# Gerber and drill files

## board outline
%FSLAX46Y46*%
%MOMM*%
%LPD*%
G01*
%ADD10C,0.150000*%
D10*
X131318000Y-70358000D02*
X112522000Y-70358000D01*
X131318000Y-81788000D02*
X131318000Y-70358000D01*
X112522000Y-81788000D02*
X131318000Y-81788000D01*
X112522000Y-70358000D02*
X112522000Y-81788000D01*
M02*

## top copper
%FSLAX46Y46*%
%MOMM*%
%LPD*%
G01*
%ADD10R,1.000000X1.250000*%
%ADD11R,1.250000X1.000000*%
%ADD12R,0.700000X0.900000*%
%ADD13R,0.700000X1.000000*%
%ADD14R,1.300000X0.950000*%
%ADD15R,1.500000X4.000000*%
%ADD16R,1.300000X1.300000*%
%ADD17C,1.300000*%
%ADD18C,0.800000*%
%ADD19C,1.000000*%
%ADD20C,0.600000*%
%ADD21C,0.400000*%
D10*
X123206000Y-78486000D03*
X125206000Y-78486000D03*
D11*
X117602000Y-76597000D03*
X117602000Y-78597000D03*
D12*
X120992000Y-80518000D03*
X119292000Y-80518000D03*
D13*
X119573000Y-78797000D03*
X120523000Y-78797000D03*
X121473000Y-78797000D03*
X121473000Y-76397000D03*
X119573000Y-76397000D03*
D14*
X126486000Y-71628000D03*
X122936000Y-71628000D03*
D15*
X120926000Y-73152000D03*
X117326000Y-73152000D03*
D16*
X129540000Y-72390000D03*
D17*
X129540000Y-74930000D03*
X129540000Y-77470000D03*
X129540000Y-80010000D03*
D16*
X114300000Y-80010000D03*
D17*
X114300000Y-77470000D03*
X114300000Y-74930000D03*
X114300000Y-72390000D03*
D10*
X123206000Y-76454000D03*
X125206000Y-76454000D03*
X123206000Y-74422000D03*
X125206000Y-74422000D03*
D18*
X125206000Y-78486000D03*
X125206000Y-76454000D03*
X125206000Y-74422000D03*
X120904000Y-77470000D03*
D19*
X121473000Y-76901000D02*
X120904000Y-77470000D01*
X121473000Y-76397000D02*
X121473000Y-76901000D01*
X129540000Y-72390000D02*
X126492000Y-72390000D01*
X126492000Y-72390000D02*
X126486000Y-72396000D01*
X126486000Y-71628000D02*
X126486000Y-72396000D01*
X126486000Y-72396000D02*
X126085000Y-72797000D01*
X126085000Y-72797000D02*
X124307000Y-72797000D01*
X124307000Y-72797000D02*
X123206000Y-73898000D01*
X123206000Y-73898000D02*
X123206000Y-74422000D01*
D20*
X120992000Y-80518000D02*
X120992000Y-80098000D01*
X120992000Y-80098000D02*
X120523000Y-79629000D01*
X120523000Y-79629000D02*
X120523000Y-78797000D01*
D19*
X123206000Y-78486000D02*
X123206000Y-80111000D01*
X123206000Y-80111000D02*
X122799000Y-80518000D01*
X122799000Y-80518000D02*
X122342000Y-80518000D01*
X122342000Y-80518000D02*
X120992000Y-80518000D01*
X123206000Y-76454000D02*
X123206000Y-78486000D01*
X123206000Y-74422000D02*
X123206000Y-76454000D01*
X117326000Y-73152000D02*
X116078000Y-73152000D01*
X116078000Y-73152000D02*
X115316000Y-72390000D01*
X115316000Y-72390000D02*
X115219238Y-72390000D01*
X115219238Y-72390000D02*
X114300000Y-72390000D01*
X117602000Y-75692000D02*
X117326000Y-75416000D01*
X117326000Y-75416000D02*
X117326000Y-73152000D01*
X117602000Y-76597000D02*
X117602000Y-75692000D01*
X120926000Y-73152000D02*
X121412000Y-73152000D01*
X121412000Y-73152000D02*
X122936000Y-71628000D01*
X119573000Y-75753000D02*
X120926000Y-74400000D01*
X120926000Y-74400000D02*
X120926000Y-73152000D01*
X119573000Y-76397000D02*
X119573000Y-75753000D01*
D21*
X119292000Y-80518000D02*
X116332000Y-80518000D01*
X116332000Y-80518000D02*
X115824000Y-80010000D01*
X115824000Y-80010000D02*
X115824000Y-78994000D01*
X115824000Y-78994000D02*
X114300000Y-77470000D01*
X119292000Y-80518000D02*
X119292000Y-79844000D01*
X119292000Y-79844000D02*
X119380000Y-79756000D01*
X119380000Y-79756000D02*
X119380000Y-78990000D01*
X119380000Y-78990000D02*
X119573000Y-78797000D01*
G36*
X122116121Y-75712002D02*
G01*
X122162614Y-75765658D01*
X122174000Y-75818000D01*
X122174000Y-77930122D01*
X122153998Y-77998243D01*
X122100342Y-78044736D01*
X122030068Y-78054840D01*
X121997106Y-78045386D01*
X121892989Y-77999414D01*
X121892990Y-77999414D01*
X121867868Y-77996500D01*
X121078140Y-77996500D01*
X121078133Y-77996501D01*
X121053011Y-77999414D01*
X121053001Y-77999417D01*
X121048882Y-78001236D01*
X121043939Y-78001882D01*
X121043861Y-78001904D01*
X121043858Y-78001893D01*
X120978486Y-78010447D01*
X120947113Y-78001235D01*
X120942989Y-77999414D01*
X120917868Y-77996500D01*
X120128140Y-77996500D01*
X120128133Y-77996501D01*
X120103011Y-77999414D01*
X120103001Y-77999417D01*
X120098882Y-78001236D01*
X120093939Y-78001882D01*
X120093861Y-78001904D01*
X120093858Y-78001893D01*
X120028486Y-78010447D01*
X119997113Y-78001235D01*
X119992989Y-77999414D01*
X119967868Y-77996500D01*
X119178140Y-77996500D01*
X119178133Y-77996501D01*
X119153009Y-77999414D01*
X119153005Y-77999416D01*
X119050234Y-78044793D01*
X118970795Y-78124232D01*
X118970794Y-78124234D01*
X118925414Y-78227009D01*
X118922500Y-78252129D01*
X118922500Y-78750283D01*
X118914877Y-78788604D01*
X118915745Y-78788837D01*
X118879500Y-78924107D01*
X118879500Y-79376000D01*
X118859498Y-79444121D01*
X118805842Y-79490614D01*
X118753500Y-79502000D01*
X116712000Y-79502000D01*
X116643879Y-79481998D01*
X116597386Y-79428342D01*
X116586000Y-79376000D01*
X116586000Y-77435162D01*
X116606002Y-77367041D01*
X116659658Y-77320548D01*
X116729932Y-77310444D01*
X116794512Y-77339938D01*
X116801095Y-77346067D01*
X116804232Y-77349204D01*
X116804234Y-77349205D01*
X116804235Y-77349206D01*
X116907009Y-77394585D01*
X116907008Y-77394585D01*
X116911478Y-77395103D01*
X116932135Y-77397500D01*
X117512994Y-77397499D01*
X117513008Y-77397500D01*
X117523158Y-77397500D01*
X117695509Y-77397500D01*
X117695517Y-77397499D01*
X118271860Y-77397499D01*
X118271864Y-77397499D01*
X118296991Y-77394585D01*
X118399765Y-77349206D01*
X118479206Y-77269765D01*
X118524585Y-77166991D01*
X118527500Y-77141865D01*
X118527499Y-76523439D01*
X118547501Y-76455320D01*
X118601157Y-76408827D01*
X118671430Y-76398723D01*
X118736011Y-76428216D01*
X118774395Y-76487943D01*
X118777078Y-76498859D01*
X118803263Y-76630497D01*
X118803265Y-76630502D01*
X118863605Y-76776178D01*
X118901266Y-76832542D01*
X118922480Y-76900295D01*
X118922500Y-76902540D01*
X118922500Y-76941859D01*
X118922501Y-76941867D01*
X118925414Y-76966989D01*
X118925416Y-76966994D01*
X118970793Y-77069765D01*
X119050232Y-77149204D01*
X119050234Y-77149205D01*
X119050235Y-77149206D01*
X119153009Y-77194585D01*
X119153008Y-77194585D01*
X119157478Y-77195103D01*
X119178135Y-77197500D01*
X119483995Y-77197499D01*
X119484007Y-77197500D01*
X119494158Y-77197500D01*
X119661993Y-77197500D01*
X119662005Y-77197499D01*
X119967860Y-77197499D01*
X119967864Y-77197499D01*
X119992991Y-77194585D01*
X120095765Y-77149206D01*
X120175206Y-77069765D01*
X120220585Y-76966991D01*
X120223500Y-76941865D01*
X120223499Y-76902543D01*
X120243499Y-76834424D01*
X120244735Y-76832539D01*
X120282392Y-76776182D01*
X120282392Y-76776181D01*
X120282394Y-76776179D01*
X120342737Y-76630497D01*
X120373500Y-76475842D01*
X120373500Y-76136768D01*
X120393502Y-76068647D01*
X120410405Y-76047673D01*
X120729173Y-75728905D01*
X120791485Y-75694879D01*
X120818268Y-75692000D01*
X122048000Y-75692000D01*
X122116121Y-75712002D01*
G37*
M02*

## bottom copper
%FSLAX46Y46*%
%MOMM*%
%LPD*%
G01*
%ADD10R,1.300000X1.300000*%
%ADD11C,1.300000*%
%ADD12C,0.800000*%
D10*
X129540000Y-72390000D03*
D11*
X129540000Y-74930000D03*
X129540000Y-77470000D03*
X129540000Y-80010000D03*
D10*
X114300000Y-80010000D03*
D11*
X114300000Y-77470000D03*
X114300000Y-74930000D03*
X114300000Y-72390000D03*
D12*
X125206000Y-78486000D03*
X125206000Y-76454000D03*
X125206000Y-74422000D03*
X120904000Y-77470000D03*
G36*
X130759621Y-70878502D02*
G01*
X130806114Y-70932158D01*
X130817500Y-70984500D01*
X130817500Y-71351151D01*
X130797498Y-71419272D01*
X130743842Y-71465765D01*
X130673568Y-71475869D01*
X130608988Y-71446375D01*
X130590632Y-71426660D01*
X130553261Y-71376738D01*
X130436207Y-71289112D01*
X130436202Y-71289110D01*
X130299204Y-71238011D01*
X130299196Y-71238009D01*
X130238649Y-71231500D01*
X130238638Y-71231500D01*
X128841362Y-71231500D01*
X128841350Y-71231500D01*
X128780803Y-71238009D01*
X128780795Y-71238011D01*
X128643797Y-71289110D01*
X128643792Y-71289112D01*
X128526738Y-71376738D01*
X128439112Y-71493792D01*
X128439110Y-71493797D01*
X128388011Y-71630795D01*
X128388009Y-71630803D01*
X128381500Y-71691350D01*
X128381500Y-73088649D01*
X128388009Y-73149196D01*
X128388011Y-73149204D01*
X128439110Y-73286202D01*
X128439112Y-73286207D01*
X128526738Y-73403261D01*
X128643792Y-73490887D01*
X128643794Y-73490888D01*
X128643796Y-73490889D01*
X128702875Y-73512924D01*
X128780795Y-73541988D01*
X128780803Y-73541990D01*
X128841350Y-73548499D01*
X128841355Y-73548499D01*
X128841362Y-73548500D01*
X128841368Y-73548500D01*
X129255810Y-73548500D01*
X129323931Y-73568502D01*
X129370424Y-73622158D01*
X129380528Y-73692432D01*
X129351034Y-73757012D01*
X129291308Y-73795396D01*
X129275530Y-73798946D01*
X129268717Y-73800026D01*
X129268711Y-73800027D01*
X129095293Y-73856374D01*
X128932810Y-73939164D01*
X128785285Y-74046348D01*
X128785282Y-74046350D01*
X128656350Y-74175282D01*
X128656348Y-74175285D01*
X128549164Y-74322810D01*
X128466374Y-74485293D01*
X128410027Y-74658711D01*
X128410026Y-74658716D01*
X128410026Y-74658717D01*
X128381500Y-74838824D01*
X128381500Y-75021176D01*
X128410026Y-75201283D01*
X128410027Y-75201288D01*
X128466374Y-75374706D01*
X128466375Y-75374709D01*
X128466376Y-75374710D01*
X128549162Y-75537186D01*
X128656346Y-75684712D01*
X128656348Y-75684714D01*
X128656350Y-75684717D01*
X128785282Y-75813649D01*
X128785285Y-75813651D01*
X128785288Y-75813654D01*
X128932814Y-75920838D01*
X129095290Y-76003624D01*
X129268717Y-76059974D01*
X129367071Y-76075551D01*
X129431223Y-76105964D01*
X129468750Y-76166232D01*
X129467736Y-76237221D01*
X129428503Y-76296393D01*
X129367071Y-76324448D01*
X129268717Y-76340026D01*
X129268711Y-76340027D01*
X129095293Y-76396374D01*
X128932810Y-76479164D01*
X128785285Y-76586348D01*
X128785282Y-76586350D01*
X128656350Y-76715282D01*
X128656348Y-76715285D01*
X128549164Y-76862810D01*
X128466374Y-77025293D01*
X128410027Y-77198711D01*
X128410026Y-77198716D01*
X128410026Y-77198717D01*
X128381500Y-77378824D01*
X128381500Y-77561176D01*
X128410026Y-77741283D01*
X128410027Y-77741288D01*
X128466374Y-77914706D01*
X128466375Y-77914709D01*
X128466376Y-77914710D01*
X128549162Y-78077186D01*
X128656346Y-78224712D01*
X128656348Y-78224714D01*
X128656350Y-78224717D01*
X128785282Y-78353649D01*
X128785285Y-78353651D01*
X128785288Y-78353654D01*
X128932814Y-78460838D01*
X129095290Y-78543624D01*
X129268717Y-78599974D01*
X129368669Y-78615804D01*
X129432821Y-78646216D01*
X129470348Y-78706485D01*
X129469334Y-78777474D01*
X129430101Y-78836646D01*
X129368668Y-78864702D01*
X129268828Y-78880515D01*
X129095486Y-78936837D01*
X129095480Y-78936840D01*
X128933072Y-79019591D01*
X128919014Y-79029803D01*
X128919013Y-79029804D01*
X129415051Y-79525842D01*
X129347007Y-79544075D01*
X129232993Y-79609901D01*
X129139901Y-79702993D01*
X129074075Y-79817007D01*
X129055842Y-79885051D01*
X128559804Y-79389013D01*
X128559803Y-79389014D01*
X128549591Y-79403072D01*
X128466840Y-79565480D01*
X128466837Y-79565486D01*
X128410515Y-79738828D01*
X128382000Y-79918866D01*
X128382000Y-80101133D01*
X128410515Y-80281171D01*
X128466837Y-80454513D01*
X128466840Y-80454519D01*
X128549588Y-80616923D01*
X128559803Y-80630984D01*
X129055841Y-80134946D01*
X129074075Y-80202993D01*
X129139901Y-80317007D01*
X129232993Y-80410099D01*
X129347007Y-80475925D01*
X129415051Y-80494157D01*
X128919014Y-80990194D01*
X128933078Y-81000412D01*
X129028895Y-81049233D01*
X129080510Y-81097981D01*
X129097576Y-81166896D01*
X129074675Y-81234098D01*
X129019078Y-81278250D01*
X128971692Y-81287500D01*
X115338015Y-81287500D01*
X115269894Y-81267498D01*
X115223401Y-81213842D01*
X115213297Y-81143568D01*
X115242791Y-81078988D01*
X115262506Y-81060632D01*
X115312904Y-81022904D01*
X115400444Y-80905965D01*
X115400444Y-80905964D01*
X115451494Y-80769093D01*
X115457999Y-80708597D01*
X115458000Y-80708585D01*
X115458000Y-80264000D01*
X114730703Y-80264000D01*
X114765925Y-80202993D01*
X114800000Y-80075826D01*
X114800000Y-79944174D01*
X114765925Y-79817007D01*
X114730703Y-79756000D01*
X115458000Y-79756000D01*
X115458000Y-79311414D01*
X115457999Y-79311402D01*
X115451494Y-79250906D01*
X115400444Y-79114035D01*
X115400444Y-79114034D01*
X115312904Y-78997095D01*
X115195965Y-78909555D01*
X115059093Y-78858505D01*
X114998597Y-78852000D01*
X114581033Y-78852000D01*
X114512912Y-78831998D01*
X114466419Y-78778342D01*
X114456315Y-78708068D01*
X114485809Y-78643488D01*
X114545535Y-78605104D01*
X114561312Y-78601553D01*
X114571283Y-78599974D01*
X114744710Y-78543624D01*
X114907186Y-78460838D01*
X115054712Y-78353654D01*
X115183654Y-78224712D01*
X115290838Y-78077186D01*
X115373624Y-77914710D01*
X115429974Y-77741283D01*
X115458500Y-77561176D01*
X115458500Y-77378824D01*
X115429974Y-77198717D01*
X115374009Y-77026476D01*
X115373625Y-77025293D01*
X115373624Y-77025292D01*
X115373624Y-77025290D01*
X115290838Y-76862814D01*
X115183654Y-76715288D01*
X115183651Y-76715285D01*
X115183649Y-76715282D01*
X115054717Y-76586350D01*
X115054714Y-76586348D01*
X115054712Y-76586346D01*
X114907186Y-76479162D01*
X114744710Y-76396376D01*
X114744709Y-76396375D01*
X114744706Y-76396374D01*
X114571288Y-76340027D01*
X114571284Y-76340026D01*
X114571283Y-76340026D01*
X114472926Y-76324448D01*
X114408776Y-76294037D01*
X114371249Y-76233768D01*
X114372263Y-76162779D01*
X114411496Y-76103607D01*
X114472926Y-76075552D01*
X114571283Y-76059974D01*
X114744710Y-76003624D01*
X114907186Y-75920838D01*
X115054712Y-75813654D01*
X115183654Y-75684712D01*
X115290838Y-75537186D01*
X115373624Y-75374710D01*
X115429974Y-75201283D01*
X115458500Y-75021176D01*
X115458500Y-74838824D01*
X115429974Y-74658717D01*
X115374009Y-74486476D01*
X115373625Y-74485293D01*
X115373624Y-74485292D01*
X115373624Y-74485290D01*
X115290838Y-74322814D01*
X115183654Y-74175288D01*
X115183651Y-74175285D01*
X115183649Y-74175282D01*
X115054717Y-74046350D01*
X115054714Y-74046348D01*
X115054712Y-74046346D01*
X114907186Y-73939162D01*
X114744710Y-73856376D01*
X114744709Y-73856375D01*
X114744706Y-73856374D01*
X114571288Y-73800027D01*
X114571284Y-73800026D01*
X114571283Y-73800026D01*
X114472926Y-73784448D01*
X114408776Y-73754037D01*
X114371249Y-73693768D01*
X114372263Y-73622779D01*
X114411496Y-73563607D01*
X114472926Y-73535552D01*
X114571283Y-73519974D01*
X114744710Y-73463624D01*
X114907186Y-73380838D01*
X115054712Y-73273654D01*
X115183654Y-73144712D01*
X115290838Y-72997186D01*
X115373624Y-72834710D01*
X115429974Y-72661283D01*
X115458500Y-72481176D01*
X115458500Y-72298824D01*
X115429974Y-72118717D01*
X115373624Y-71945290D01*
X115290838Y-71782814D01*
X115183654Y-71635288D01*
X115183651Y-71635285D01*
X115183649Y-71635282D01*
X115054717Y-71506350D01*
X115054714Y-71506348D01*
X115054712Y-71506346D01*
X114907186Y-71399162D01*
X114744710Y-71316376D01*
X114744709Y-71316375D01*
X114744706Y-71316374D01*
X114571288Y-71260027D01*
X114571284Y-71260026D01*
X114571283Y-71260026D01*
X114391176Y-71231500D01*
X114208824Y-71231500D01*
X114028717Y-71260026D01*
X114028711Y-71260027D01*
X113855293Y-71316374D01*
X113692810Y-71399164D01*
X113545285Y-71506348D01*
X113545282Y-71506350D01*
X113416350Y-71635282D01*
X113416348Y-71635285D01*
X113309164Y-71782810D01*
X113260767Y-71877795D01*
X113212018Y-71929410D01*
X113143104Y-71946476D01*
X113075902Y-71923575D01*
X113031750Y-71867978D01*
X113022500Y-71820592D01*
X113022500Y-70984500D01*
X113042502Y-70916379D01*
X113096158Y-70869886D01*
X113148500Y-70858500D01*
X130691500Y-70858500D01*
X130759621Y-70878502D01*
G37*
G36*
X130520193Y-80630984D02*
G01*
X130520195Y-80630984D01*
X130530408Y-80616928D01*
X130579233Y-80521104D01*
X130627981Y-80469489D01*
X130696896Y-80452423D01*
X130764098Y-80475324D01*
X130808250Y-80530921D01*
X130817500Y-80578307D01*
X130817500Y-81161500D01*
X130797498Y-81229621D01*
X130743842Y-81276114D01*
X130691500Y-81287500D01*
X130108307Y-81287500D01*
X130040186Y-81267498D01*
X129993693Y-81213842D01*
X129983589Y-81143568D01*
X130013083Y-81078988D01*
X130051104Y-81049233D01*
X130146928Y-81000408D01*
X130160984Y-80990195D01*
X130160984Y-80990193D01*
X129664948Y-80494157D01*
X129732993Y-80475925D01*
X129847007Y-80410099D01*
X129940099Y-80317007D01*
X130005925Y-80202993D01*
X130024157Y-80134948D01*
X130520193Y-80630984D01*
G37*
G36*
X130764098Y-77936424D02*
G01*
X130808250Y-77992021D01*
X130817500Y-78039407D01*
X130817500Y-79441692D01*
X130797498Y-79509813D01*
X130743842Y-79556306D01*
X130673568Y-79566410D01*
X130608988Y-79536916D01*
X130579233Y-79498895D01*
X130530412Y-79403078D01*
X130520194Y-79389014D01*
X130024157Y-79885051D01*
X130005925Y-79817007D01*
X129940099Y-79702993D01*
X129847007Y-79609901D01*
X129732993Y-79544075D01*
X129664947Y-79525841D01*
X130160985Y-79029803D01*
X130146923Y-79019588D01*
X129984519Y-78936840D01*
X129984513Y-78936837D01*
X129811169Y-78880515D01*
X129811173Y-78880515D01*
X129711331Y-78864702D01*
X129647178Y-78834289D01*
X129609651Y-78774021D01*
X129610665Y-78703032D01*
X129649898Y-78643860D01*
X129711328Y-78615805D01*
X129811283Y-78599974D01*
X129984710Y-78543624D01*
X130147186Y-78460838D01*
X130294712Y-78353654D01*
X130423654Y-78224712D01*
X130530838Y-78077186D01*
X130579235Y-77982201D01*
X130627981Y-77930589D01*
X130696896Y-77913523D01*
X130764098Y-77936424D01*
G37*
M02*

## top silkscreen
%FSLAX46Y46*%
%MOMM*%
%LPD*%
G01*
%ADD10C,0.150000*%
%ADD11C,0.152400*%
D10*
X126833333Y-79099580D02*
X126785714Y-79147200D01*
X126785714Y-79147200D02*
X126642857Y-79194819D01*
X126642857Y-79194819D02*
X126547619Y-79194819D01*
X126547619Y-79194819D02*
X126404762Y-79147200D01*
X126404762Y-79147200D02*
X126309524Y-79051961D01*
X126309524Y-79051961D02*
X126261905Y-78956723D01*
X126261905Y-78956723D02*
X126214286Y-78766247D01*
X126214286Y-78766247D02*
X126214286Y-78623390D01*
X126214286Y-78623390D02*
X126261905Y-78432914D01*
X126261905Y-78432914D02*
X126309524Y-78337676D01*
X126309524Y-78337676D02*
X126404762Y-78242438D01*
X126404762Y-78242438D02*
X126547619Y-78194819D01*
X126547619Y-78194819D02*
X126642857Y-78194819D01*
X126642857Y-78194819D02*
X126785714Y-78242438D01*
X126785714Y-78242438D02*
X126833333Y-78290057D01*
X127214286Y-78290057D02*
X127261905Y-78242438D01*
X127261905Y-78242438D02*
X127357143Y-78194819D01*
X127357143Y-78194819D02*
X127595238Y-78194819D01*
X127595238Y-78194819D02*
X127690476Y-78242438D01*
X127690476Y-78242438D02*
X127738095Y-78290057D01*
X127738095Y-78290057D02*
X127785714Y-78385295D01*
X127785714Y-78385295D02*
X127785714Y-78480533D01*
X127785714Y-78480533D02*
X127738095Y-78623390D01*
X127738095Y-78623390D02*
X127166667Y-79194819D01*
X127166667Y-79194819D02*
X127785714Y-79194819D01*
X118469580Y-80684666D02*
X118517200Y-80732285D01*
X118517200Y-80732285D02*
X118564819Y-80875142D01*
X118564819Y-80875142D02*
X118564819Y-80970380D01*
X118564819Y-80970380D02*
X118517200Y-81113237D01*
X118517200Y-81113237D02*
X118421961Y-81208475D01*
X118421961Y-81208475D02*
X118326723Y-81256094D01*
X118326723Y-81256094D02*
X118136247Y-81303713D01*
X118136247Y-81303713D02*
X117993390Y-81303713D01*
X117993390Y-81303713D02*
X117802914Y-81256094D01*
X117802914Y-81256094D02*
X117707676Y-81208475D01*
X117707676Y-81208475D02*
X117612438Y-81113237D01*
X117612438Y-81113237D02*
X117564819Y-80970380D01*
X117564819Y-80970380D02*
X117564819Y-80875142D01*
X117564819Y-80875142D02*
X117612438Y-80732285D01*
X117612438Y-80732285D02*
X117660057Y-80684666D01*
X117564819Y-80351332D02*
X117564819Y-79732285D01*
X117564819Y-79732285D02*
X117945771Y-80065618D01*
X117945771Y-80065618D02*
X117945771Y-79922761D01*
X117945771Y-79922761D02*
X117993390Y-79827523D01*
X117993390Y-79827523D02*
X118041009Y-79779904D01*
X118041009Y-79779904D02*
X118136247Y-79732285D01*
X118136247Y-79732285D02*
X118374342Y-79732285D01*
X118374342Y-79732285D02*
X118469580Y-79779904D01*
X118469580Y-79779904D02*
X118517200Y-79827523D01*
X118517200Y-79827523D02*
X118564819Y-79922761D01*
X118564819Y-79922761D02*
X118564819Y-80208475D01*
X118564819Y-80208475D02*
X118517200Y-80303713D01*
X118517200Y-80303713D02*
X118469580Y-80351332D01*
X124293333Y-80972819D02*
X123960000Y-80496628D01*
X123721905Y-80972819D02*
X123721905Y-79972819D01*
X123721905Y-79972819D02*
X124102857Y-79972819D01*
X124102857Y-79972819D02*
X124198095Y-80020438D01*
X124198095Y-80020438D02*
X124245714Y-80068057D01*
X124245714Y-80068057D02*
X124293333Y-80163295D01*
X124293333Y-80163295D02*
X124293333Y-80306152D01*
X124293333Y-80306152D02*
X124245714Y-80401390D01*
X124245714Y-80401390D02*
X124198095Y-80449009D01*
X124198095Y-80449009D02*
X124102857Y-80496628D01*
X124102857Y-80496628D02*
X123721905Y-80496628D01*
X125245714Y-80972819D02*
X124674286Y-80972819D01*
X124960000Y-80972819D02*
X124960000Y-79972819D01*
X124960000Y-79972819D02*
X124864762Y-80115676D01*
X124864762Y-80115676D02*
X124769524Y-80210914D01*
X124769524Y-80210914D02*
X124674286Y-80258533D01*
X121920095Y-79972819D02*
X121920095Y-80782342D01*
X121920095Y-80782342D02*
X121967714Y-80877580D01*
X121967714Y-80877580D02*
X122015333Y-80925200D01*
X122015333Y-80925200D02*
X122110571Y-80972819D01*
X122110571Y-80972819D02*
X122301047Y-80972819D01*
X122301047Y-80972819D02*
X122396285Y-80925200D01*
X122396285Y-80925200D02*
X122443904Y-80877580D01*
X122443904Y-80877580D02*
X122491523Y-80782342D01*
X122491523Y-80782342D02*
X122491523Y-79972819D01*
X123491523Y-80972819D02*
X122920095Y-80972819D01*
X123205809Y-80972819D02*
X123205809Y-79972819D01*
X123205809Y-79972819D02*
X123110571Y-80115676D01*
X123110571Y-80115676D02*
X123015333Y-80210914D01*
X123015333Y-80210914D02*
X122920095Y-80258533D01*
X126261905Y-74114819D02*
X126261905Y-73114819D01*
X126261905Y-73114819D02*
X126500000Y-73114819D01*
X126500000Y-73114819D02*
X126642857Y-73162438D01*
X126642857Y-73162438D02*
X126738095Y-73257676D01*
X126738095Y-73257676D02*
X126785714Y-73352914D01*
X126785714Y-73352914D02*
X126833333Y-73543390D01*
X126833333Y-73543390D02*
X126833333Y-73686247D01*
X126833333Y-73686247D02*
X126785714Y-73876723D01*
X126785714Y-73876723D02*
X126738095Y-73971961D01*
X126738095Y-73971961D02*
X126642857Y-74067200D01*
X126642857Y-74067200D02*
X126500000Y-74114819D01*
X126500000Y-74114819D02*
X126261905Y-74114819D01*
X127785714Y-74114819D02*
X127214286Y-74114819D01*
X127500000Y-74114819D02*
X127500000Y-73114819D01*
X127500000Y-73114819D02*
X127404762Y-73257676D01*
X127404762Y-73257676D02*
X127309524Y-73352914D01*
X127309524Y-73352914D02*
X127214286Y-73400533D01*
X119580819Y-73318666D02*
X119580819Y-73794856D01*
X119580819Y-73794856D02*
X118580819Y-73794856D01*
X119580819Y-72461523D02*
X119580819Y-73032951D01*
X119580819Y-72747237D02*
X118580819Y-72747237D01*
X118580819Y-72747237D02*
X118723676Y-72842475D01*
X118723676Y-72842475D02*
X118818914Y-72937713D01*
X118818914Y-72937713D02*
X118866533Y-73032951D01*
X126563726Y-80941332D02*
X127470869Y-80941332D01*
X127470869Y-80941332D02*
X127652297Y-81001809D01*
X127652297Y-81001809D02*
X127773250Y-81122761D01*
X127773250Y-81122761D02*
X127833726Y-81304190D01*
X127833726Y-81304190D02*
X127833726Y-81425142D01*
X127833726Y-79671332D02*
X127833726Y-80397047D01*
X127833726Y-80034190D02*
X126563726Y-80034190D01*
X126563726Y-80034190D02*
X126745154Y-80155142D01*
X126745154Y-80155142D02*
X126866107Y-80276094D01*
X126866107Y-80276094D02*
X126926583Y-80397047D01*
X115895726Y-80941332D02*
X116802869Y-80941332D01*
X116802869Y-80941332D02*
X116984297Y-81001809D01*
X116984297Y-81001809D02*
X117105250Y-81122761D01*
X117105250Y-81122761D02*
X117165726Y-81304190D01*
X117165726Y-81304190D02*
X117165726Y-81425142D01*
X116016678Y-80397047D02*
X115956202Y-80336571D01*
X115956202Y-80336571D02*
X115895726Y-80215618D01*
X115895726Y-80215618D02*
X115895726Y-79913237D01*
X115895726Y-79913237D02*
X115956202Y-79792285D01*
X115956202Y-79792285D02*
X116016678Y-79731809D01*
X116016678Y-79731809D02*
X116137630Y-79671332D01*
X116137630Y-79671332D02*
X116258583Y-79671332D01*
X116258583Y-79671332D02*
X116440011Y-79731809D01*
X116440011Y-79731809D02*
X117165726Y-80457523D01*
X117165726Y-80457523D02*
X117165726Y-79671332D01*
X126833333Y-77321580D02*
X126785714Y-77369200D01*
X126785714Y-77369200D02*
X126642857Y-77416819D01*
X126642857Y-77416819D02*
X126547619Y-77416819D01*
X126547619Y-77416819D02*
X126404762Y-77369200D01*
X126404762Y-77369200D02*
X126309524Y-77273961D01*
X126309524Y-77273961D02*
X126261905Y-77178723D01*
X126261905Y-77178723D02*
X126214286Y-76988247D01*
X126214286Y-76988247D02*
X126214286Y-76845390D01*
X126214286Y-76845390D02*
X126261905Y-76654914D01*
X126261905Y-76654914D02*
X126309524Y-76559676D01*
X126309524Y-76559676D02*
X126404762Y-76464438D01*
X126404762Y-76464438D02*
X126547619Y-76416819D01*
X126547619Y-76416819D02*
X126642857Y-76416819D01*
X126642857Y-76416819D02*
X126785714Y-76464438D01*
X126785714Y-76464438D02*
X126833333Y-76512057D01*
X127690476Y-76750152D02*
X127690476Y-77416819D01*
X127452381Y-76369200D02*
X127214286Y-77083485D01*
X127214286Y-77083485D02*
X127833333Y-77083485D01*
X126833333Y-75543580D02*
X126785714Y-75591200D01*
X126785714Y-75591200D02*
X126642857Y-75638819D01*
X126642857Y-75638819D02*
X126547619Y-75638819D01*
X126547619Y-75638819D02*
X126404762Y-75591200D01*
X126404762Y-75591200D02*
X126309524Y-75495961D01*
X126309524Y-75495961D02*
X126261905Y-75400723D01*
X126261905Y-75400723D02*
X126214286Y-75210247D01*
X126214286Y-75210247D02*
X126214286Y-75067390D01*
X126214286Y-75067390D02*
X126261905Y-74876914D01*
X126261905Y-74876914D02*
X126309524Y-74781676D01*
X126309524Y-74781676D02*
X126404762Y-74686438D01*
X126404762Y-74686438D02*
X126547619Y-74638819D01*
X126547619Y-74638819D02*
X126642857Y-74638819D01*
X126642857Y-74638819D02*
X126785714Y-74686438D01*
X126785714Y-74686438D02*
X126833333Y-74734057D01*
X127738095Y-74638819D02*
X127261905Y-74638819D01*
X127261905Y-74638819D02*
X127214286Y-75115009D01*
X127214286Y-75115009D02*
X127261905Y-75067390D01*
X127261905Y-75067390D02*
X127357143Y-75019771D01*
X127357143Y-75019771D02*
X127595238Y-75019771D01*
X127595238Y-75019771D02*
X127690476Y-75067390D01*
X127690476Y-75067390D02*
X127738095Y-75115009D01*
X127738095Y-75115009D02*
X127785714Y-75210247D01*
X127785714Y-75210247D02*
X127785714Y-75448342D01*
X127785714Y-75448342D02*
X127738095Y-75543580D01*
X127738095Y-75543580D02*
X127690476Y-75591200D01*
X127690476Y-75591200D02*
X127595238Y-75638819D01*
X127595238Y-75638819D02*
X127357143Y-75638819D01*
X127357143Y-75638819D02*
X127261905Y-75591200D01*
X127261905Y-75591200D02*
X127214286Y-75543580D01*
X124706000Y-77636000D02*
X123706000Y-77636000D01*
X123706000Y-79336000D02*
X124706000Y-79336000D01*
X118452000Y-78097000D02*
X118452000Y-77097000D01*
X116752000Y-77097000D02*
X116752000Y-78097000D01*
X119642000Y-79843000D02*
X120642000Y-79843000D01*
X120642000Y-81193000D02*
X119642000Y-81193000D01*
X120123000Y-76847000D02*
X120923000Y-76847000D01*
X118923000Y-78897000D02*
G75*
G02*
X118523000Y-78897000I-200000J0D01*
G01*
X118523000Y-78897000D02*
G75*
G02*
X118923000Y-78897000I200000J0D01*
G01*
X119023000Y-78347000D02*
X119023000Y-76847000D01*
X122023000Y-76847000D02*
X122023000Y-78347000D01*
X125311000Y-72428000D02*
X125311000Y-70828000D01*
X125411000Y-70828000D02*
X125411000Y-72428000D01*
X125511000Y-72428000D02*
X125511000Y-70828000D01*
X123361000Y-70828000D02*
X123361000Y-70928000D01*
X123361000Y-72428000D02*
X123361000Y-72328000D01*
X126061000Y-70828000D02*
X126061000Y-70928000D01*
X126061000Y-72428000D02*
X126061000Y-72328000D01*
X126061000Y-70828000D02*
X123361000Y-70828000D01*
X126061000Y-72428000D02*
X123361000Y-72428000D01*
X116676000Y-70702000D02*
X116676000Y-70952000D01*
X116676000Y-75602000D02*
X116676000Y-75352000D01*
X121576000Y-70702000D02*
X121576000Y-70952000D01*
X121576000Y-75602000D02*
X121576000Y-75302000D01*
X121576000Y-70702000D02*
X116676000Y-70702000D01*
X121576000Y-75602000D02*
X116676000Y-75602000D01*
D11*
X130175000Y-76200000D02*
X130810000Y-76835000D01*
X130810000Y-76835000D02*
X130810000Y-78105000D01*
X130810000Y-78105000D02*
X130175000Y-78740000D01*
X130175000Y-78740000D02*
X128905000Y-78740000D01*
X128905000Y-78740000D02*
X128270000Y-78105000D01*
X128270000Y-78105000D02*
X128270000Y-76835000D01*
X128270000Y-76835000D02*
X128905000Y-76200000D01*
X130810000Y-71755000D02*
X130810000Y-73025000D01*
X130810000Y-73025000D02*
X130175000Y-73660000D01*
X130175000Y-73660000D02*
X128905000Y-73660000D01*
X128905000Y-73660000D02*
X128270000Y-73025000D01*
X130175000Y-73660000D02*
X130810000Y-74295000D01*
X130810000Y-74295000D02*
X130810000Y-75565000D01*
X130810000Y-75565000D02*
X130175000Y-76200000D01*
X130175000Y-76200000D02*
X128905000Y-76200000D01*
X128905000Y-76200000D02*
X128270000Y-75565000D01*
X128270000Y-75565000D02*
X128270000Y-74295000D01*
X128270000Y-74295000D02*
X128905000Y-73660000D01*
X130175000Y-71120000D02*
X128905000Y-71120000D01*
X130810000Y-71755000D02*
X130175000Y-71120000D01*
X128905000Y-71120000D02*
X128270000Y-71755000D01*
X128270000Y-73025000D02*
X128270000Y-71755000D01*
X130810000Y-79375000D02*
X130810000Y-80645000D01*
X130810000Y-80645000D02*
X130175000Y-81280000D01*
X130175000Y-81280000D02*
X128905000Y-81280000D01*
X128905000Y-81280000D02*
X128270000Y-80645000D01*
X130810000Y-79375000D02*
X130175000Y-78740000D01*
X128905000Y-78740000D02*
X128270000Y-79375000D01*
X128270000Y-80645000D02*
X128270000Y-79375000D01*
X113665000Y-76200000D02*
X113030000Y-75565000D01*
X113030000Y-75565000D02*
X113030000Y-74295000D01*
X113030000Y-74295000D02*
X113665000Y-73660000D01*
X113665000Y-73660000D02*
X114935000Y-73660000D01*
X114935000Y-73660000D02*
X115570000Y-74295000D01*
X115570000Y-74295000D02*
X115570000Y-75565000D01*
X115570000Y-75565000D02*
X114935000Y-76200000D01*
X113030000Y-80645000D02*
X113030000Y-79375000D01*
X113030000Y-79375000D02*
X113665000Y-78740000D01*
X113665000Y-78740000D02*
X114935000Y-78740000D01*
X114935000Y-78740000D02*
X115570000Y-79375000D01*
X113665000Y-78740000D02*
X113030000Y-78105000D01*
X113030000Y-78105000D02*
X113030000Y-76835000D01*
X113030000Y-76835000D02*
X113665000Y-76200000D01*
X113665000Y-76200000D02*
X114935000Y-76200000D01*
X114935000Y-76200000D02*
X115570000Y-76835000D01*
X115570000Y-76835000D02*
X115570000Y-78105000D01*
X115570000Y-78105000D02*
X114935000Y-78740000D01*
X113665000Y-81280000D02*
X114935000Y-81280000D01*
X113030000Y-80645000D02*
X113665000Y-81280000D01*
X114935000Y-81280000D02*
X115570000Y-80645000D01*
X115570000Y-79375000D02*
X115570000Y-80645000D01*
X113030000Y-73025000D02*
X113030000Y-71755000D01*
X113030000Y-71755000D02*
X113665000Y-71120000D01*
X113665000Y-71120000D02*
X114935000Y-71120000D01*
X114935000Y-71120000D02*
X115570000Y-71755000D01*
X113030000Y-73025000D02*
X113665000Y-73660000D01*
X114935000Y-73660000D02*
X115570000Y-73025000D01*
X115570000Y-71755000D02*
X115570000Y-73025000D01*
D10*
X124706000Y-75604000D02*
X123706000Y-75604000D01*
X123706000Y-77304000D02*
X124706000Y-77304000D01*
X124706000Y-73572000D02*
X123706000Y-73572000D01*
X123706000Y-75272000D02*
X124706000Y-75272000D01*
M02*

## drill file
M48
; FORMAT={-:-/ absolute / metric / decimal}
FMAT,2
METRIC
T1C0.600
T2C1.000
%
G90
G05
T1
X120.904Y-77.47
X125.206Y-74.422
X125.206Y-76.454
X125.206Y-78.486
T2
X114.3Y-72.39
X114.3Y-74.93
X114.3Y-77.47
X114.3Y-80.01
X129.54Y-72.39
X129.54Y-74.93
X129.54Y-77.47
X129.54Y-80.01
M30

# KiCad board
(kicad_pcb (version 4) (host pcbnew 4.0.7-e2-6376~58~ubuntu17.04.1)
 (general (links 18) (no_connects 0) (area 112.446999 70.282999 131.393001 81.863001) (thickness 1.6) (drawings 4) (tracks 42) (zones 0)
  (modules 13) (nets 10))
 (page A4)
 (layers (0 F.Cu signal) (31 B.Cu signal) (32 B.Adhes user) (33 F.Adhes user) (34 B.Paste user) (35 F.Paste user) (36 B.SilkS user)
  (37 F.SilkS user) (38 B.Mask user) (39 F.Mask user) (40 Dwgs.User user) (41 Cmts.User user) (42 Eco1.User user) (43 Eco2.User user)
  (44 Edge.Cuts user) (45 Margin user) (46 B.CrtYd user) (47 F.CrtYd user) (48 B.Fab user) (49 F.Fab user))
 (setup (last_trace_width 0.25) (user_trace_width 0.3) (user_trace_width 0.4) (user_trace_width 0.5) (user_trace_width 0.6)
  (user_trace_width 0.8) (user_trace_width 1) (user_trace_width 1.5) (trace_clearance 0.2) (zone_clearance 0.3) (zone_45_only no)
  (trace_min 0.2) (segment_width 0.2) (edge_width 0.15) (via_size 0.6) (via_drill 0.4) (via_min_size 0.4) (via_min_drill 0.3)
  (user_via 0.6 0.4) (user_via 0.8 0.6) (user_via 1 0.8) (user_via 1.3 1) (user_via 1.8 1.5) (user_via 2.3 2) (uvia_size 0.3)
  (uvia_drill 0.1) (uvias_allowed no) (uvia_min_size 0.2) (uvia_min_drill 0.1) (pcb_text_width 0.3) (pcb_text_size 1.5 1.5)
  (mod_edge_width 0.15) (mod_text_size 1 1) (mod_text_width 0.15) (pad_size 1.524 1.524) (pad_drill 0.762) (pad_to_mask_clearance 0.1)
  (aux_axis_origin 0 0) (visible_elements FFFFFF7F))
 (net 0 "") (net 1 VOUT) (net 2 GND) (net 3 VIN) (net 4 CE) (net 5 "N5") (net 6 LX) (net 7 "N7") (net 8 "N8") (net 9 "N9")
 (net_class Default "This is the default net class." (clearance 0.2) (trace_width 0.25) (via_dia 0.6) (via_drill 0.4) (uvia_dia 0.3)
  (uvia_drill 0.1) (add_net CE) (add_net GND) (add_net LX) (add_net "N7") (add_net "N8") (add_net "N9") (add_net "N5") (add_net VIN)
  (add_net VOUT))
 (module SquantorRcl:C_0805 (layer F.Cu) (at 124.206 78.486)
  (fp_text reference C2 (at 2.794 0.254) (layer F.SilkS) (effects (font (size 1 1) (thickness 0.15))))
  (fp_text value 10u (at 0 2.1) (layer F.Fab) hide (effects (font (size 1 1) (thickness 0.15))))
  (fp_line (start 0.5 -0.85) (end -0.5 -0.85) (layer F.SilkS) (width 0.15))
  (fp_line (start -0.5 0.85) (end 0.5 0.85) (layer F.SilkS) (width 0.15))
  (pad 1 smd rect (at -1 0) (size 1 1.25) (layers F.Cu F.Paste F.Mask) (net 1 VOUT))
  (pad 2 smd rect (at 1 0) (size 1 1.25) (layers F.Cu F.Paste F.Mask) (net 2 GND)))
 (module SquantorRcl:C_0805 (layer F.Cu) (at 117.602 77.597 270)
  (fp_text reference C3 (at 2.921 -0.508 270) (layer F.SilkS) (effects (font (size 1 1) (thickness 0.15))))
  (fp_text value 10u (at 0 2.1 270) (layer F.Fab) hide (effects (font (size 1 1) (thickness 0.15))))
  (fp_line (start 0.5 -0.85) (end -0.5 -0.85) (layer F.SilkS) (width 0.15))
  (fp_line (start -0.5 0.85) (end 0.5 0.85) (layer F.SilkS) (width 0.15))
  (pad 1 smd rect (at -1 0 270) (size 1 1.25) (layers F.Cu F.Paste F.Mask) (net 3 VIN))
  (pad 2 smd rect (at 1 0 270) (size 1 1.25) (layers F.Cu F.Paste F.Mask) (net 2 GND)))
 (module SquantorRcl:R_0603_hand (layer F.Cu) (at 120.142 80.518 180)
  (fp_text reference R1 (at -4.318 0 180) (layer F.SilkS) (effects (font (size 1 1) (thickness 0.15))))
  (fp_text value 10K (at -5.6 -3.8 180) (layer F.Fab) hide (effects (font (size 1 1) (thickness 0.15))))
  (fp_line (start 0.5 0.675) (end -0.5 0.675) (layer F.SilkS) (width 0.15))
  (fp_line (start -0.5 -0.675) (end 0.5 -0.675) (layer F.SilkS) (width 0.15))
  (pad 1 smd rect (at -0.85 0 180) (size 0.7 0.9) (layers F.Cu F.Paste F.Mask) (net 1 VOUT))
  (pad 2 smd rect (at 0.85 0 180) (size 0.7 0.9) (layers F.Cu F.Paste F.Mask) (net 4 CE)))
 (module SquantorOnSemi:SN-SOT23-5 (layer F.Cu) (at 120.523 77.597)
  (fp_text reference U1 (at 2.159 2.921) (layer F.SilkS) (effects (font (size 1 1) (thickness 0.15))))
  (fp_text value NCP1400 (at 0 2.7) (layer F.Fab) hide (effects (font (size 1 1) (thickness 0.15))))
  (fp_line (start -0.4 -0.75) (end 0.4 -0.75) (layer F.SilkS) (width 0.15))
  (fp_circle (center -1.8 1.3) (end -1.6 1.3) (layer F.SilkS) (width 0.15))
  (fp_line (start -1.5 0.75) (end -1.5 -0.75) (layer F.SilkS) (width 0.15))
  (fp_line (start 1.5 -0.75) (end 1.5 0.75) (layer F.SilkS) (width 0.15))
  (pad 1 smd rect (at -0.95 1.2) (size 0.7 1) (layers F.Cu F.Paste F.Mask) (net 4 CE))
  (pad 2 smd rect (at 0 1.2) (size 0.7 1) (layers F.Cu F.Paste F.Mask) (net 1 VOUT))
  (pad 3 smd rect (at 0.95 1.2) (size 0.7 1) (layers F.Cu F.Paste F.Mask) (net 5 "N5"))
  (pad 4 smd rect (at 0.95 -1.2) (size 0.7 1) (layers F.Cu F.Paste F.Mask) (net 2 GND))
  (pad 5 smd rect (at -0.95 -1.2) (size 0.7 1) (layers F.Cu F.Paste F.Mask) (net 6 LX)))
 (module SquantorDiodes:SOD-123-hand (layer F.Cu) (at 124.711 71.628 180)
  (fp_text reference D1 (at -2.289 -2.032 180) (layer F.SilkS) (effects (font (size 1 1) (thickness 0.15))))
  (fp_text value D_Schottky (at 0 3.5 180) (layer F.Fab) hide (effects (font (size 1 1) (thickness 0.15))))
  (fp_line (start -0.6 -0.8) (end -0.6 0.8) (layer F.SilkS) (width 0.15))
  (fp_line (start -0.7 0.8) (end -0.7 -0.8) (layer F.SilkS) (width 0.15))
  (fp_line (start -0.8 -0.8) (end -0.8 0.8) (layer F.SilkS) (width 0.15))
  (fp_line (start 1.35 0.8) (end 1.35 0.7) (layer F.SilkS) (width 0.15))
  (fp_line (start 1.35 -0.8) (end 1.35 -0.7) (layer F.SilkS) (width 0.15))
  (fp_line (start -1.35 0.8) (end -1.35 0.7) (layer F.SilkS) (width 0.15))
  (fp_line (start -1.35 -0.8) (end -1.35 -0.7) (layer F.SilkS) (width 0.15))
  (fp_line (start -1.35 0.8) (end 1.35 0.8) (layer F.SilkS) (width 0.15))
  (fp_line (start -1.35 -0.8) (end 1.35 -0.8) (layer F.SilkS) (width 0.15))
  (pad 1 smd rect (at -1.775 0 180) (size 1.3 0.95) (layers F.Cu F.Paste F.Mask) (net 1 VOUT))
  (pad 2 smd rect (at 1.775 0 180) (size 1.3 0.95) (layers F.Cu F.Paste F.Mask) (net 6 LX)))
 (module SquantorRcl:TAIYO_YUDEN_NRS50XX (layer F.Cu) (at 119.126 73.152 180)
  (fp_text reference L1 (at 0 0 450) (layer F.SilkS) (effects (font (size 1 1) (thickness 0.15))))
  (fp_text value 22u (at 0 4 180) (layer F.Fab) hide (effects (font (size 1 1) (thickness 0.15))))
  (fp_line (start 2.45 2.45) (end 2.45 2.2) (layer F.SilkS) (width 0.15))
  (fp_line (start 2.45 -2.45) (end 2.45 -2.2) (layer F.SilkS) (width 0.15))
  (fp_line (start -2.45 2.45) (end -2.45 2.2) (layer F.SilkS) (width 0.15))
  (fp_line (start -2.45 -2.45) (end -2.45 -2.15) (layer F.SilkS) (width 0.15))
  (fp_line (start -2.45 2.45) (end 2.45 2.45) (layer F.SilkS) (width 0.15))
  (fp_line (start -2.45 -2.45) (end 2.45 -2.45) (layer F.SilkS) (width 0.15))
  (pad 1 smd rect (at -1.8 0 180) (size 1.5 4) (layers F.Cu F.Paste F.Mask) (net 6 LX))
  (pad 2 smd rect (at 1.8 0 180) (size 1.5 4) (layers F.Cu F.Paste F.Mask) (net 3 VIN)))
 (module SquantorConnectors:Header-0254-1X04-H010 (layer F.Cu) (at 129.54 76.2 270)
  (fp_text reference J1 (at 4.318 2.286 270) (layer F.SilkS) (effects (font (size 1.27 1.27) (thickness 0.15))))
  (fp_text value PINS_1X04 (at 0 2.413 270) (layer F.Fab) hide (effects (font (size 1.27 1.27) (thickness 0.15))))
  (fp_line (start 0 -0.635) (end 0.635 -1.27) (layer F.SilkS) (width 0.1524))
  (fp_line (start 0.635 -1.27) (end 1.905 -1.27) (layer F.SilkS) (width 0.1524))
  (fp_line (start 1.905 -1.27) (end 2.54 -0.635) (layer F.SilkS) (width 0.1524))
  (fp_line (start 2.54 -0.635) (end 2.54 0.635) (layer F.SilkS) (width 0.1524))
  (fp_line (start 2.54 0.635) (end 1.905 1.27) (layer F.SilkS) (width 0.1524))
  (fp_line (start 1.905 1.27) (end 0.635 1.27) (layer F.SilkS) (width 0.1524))
  (fp_line (start 0.635 1.27) (end 0 0.635) (layer F.SilkS) (width 0.1524))
  (fp_line (start -4.445 -1.27) (end -3.175 -1.27) (layer F.SilkS) (width 0.1524))
  (fp_line (start -3.175 -1.27) (end -2.54 -0.635) (layer F.SilkS) (width 0.1524))
  (fp_line (start -2.54 -0.635) (end -2.54 0.635) (layer F.SilkS) (width 0.1524))
  (fp_line (start -2.54 0.635) (end -3.175 1.27) (layer F.SilkS) (width 0.1524))
  (fp_line (start -2.54 -0.635) (end -1.905 -1.27) (layer F.SilkS) (width 0.1524))
  (fp_line (start -1.905 -1.27) (end -0.635 -1.27) (layer F.SilkS) (width 0.1524))
  (fp_line (start -0.635 -1.27) (end 0 -0.635) (layer F.SilkS) (width 0.1524))
  (fp_line (start 0 -0.635) (end 0 0.635) (layer F.SilkS) (width 0.1524))
  (fp_line (start 0 0.635) (end -0.635 1.27) (layer F.SilkS) (width 0.1524))
  (fp_line (start -0.635 1.27) (end -1.905 1.27) (layer F.SilkS) (width 0.1524))
  (fp_line (start -1.905 1.27) (end -2.54 0.635) (layer F.SilkS) (width 0.1524))
  (fp_line (start -5.08 -0.635) (end -5.08 0.635) (layer F.SilkS) (width 0.1524))
  (fp_line (start -4.445 -1.27) (end -5.08 -0.635) (layer F.SilkS) (width 0.1524))
  (fp_line (start -5.08 0.635) (end -4.445 1.27) (layer F.SilkS) (width 0.1524))
  (fp_line (start -3.175 1.27) (end -4.445 1.27) (layer F.SilkS) (width 0.1524))
  (fp_line (start 3.175 -1.27) (end 4.445 -1.27) (layer F.SilkS) (width 0.1524))
  (fp_line (start 4.445 -1.27) (end 5.08 -0.635) (layer F.SilkS) (width 0.1524))
  (fp_line (start 5.08 -0.635) (end 5.08 0.635) (layer F.SilkS) (width 0.1524))
  (fp_line (start 5.08 0.635) (end 4.445 1.27) (layer F.SilkS) (width 0.1524))
  (fp_line (start 3.175 -1.27) (end 2.54 -0.635) (layer F.SilkS) (width 0.1524))
  (fp_line (start 2.54 0.635) (end 3.175 1.27) (layer F.SilkS) (width 0.1524))
  (fp_line (start 4.445 1.27) (end 3.175 1.27) (layer F.SilkS) (width 0.1524))
  (pad 1 thru_hole rect (at -3.81 0 90) (size 1.3 1.3) (drill 1) (layers *.Cu *.Mask) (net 1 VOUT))
  (pad 2 thru_hole circle (at -1.27 0 90) (size 1.3 1.3) (drill 1) (layers *.Cu *.Mask) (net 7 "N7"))
  (pad 3 thru_hole circle (at 1.27 0 90) (size 1.3 1.3) (drill 1) (layers *.Cu *.Mask) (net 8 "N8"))
  (pad 4 thru_hole circle (at 3.81 0 90) (size 1.3 1.3) (drill 1) (layers *.Cu *.Mask) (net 2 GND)))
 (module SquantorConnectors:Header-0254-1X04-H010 (layer F.Cu) (at 114.3 76.2 90)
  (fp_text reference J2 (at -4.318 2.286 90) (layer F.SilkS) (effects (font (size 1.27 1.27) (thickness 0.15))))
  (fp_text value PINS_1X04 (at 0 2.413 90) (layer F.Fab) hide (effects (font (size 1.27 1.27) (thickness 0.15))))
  (fp_line (start 0 -0.635) (end 0.635 -1.27) (layer F.SilkS) (width 0.1524))
  (fp_line (start 0.635 -1.27) (end 1.905 -1.27) (layer F.SilkS) (width 0.1524))
  (fp_line (start 1.905 -1.27) (end 2.54 -0.635) (layer F.SilkS) (width 0.1524))
  (fp_line (start 2.54 -0.635) (end 2.54 0.635) (layer F.SilkS) (width 0.1524))
  (fp_line (start 2.54 0.635) (end 1.905 1.27) (layer F.SilkS) (width 0.1524))
  (fp_line (start 1.905 1.27) (end 0.635 1.27) (layer F.SilkS) (width 0.1524))
  (fp_line (start 0.635 1.27) (end 0 0.635) (layer F.SilkS) (width 0.1524))
  (fp_line (start -4.445 -1.27) (end -3.175 -1.27) (layer F.SilkS) (width 0.1524))
  (fp_line (start -3.175 -1.27) (end -2.54 -0.635) (layer F.SilkS) (width 0.1524))
  (fp_line (start -2.54 -0.635) (end -2.54 0.635) (layer F.SilkS) (width 0.1524))
  (fp_line (start -2.54 0.635) (end -3.175 1.27) (layer F.SilkS) (width 0.1524))
  (fp_line (start -2.54 -0.635) (end -1.905 -1.27) (layer F.SilkS) (width 0.1524))
  (fp_line (start -1.905 -1.27) (end -0.635 -1.27) (layer F.SilkS) (width 0.1524))
  (fp_line (start -0.635 -1.27) (end 0 -0.635) (layer F.SilkS) (width 0.1524))
  (fp_line (start 0 -0.635) (end 0 0.635) (layer F.SilkS) (width 0.1524))
  (fp_line (start 0 0.635) (end -0.635 1.27) (layer F.SilkS) (width 0.1524))
  (fp_line (start -0.635 1.27) (end -1.905 1.27) (layer F.SilkS) (width 0.1524))
  (fp_line (start -1.905 1.27) (end -2.54 0.635) (layer F.SilkS) (width 0.1524))
  (fp_line (start -5.08 -0.635) (end -5.08 0.635) (layer F.SilkS) (width 0.1524))
  (fp_line (start -4.445 -1.27) (end -5.08 -0.635) (layer F.SilkS) (width 0.1524))
  (fp_line (start -5.08 0.635) (end -4.445 1.27) (layer F.SilkS) (width 0.1524))
  (fp_line (start -3.175 1.27) (end -4.445 1.27) (layer F.SilkS) (width 0.1524))
  (fp_line (start 3.175 -1.27) (end 4.445 -1.27) (layer F.SilkS) (width 0.1524))
  (fp_line (start 4.445 -1.27) (end 5.08 -0.635) (layer F.SilkS) (width 0.1524))
  (fp_line (start 5.08 -0.635) (end 5.08 0.635) (layer F.SilkS) (width 0.1524))
  (fp_line (start 5.08 0.635) (end 4.445 1.27) (layer F.SilkS) (width 0.1524))
  (fp_line (start 3.175 -1.27) (end 2.54 -0.635) (layer F.SilkS) (width 0.1524))
  (fp_line (start 2.54 0.635) (end 3.175 1.27) (layer F.SilkS) (width 0.1524))
  (fp_line (start 4.445 1.27) (end 3.175 1.27) (layer F.SilkS) (width 0.1524))
  (pad 1 thru_hole rect (at -3.81 0 270) (size 1.3 1.3) (drill 1) (layers *.Cu *.Mask) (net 2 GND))
  (pad 2 thru_hole circle (at -1.27 0 270) (size 1.3 1.3) (drill 1) (layers *.Cu *.Mask) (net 4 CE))
  (pad 3 thru_hole circle (at 1.27 0 270) (size 1.3 1.3) (drill 1) (layers *.Cu *.Mask) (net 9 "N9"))
  (pad 4 thru_hole circle (at 3.81 0 270) (size 1.3 1.3) (drill 1) (layers *.Cu *.Mask) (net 3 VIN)))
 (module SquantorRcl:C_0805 (layer F.Cu) (at 124.206 76.454)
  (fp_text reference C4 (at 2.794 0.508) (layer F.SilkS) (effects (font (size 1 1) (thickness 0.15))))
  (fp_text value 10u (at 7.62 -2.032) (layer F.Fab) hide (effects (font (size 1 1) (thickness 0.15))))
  (fp_line (start 0.5 -0.85) (end -0.5 -0.85) (layer F.SilkS) (width 0.15))
  (fp_line (start -0.5 0.85) (end 0.5 0.85) (layer F.SilkS) (width 0.15))
  (pad 1 smd rect (at -1 0) (size 1 1.25) (layers F.Cu F.Paste F.Mask) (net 1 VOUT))
  (pad 2 smd rect (at 1 0) (size 1 1.25) (layers F.Cu F.Paste F.Mask) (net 2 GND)))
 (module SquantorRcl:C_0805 (layer F.Cu) (at 124.206 74.422)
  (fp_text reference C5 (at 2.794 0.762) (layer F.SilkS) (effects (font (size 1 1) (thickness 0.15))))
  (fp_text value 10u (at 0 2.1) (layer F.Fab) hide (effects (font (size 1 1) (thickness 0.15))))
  (fp_line (start 0.5 -0.85) (end -0.5 -0.85) (layer F.SilkS) (width 0.15))
  (fp_line (start -0.5 0.85) (end 0.5 0.85) (layer F.SilkS) (width 0.15))
  (pad 1 smd rect (at -1 0) (size 1 1.25) (layers F.Cu F.Paste F.Mask) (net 1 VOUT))
  (pad 2 smd rect (at 1 0) (size 1 1.25) (layers F.Cu F.Paste F.Mask) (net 2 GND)))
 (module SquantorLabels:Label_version (layer F.Cu) (at 119.8372 79.7052)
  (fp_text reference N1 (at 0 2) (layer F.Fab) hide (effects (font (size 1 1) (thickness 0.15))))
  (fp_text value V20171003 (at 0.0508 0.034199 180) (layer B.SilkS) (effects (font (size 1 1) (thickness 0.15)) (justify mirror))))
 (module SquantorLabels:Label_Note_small (layer B.Cu) (at 115.9764 74.7268)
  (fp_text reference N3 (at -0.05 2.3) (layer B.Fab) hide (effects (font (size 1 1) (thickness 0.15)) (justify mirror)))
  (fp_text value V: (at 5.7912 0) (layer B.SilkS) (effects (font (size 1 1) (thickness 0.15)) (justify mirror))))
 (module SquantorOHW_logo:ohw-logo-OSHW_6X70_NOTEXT (layer B.Cu) (at 119.1768 77.4192 180)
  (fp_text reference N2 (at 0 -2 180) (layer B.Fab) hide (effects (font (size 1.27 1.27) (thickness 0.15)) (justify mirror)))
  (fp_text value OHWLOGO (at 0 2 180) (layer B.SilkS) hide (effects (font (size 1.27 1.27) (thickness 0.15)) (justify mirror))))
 (gr_line (start 131.318 70.358) (end 112.522 70.358) (layer Edge.Cuts) (width 0.15))
 (gr_line (start 131.318 81.788) (end 131.318 70.358) (layer Edge.Cuts) (width 0.15))
 (gr_line (start 112.522 81.788) (end 131.318 81.788) (layer Edge.Cuts) (width 0.15))
 (gr_line (start 112.522 70.358) (end 112.522 81.788) (layer Edge.Cuts) (width 0.15))
 (via (at 125.206 78.486) (size 0.8) (drill 0.6) (layers F.Cu B.Cu) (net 2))
 (via (at 125.206 76.454) (size 0.8) (drill 0.6) (layers F.Cu B.Cu) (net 2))
 (via (at 125.206 74.422) (size 0.8) (drill 0.6) (layers F.Cu B.Cu) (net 2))
 (segment (start 121.473 76.901) (end 120.904 77.47) (width 1) (layer F.Cu) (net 2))
 (via (at 120.904 77.47) (size 0.8) (drill 0.6) (layers F.Cu B.Cu) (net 2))
 (segment (start 121.473 76.397) (end 121.473 76.901) (width 1) (layer F.Cu) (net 2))
 (segment (start 129.54 72.39) (end 126.492 72.39) (width 1) (layer F.Cu) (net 1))
 (segment (start 126.492 72.39) (end 126.486 72.396) (width 1) (layer F.Cu) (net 1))
 (segment (start 126.486 71.628) (end 126.486 72.396) (width 1) (layer F.Cu) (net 1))
 (segment (start 126.486 72.396) (end 126.085 72.797) (width 1) (layer F.Cu) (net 1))
 (segment (start 126.085 72.797) (end 124.307 72.797) (width 1) (layer F.Cu) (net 1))
 (segment (start 124.307 72.797) (end 123.206 73.898) (width 1) (layer F.Cu) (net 1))
 (segment (start 123.206 73.898) (end 123.206 74.422) (width 1) (layer F.Cu) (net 1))
 (segment (start 120.992 80.518) (end 120.992 80.098) (width 0.6) (layer F.Cu) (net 1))
 (segment (start 120.992 80.098) (end 120.523 79.629) (width 0.6) (layer F.Cu) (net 1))
 (segment (start 120.523 79.629) (end 120.523 78.797) (width 0.6) (layer F.Cu) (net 1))
 (segment (start 123.206 78.486) (end 123.206 80.111) (width 1) (layer F.Cu) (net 1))
 (segment (start 123.206 80.111) (end 122.799 80.518) (width 1) (layer F.Cu) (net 1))
 (segment (start 122.799 80.518) (end 122.342 80.518) (width 1) (layer F.Cu) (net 1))
 (segment (start 122.342 80.518) (end 120.992 80.518) (width 1) (layer F.Cu) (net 1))
 (segment (start 123.206 76.454) (end 123.206 78.486) (width 1) (layer F.Cu) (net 1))
 (segment (start 123.206 74.422) (end 123.206 76.454) (width 1) (layer F.Cu) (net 1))
 (segment (start 117.326 73.152) (end 116.078 73.152) (width 1) (layer F.Cu) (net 3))
 (segment (start 116.078 73.152) (end 115.316 72.39) (width 1) (layer F.Cu) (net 3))
 (segment (start 115.316 72.39) (end 115.219238 72.39) (width 1) (layer F.Cu) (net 3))
 (segment (start 115.219238 72.39) (end 114.3 72.39) (width 1) (layer F.Cu) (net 3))
 (segment (start 117.602 75.692) (end 117.326 75.416) (width 1) (layer F.Cu) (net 3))
 (segment (start 117.326 75.416) (end 117.326 73.152) (width 1) (layer F.Cu) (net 3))
 (segment (start 117.602 76.597) (end 117.602 75.692) (width 1) (layer F.Cu) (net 3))
 (segment (start 120.926 73.152) (end 121.412 73.152) (width 1) (layer F.Cu) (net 6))
 (segment (start 121.412 73.152) (end 122.936 71.628) (width 1) (layer F.Cu) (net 6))
 (segment (start 119.573 75.753) (end 120.926 74.4) (width 1) (layer F.Cu) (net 6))
 (segment (start 120.926 74.4) (end 120.926 73.152) (width 1) (layer F.Cu) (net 6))
 (segment (start 119.573 76.397) (end 119.573 75.753) (width 1) (layer F.Cu) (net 6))
 (segment (start 119.292 80.518) (end 116.332 80.518) (width 0.4) (layer F.Cu) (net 4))
 (segment (start 116.332 80.518) (end 115.824 80.01) (width 0.4) (layer F.Cu) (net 4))
 (segment (start 115.824 80.01) (end 115.824 78.994) (width 0.4) (layer F.Cu) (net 4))
 (segment (start 115.824 78.994) (end 114.3 77.47) (width 0.4) (layer F.Cu) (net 4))
 (segment (start 119.292 80.518) (end 119.292 79.844) (width 0.4) (layer F.Cu) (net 4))
 (segment (start 119.292 79.844) (end 119.38 79.756) (width 0.4) (layer F.Cu) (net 4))
 (segment (start 119.38 79.756) (end 119.38 78.99) (width 0.4) (layer F.Cu) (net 4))
 (segment (start 119.38 78.99) (end 119.573 78.797) (width 0.4) (layer F.Cu) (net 4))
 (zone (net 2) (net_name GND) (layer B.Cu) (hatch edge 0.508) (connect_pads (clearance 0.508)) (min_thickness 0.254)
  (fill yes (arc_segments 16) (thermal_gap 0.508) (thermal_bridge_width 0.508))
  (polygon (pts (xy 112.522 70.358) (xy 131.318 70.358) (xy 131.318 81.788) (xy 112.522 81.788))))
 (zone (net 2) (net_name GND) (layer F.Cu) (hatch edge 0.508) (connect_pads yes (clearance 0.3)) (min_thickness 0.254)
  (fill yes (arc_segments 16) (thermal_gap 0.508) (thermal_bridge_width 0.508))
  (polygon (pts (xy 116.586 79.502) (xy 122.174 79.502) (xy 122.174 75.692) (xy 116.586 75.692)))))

